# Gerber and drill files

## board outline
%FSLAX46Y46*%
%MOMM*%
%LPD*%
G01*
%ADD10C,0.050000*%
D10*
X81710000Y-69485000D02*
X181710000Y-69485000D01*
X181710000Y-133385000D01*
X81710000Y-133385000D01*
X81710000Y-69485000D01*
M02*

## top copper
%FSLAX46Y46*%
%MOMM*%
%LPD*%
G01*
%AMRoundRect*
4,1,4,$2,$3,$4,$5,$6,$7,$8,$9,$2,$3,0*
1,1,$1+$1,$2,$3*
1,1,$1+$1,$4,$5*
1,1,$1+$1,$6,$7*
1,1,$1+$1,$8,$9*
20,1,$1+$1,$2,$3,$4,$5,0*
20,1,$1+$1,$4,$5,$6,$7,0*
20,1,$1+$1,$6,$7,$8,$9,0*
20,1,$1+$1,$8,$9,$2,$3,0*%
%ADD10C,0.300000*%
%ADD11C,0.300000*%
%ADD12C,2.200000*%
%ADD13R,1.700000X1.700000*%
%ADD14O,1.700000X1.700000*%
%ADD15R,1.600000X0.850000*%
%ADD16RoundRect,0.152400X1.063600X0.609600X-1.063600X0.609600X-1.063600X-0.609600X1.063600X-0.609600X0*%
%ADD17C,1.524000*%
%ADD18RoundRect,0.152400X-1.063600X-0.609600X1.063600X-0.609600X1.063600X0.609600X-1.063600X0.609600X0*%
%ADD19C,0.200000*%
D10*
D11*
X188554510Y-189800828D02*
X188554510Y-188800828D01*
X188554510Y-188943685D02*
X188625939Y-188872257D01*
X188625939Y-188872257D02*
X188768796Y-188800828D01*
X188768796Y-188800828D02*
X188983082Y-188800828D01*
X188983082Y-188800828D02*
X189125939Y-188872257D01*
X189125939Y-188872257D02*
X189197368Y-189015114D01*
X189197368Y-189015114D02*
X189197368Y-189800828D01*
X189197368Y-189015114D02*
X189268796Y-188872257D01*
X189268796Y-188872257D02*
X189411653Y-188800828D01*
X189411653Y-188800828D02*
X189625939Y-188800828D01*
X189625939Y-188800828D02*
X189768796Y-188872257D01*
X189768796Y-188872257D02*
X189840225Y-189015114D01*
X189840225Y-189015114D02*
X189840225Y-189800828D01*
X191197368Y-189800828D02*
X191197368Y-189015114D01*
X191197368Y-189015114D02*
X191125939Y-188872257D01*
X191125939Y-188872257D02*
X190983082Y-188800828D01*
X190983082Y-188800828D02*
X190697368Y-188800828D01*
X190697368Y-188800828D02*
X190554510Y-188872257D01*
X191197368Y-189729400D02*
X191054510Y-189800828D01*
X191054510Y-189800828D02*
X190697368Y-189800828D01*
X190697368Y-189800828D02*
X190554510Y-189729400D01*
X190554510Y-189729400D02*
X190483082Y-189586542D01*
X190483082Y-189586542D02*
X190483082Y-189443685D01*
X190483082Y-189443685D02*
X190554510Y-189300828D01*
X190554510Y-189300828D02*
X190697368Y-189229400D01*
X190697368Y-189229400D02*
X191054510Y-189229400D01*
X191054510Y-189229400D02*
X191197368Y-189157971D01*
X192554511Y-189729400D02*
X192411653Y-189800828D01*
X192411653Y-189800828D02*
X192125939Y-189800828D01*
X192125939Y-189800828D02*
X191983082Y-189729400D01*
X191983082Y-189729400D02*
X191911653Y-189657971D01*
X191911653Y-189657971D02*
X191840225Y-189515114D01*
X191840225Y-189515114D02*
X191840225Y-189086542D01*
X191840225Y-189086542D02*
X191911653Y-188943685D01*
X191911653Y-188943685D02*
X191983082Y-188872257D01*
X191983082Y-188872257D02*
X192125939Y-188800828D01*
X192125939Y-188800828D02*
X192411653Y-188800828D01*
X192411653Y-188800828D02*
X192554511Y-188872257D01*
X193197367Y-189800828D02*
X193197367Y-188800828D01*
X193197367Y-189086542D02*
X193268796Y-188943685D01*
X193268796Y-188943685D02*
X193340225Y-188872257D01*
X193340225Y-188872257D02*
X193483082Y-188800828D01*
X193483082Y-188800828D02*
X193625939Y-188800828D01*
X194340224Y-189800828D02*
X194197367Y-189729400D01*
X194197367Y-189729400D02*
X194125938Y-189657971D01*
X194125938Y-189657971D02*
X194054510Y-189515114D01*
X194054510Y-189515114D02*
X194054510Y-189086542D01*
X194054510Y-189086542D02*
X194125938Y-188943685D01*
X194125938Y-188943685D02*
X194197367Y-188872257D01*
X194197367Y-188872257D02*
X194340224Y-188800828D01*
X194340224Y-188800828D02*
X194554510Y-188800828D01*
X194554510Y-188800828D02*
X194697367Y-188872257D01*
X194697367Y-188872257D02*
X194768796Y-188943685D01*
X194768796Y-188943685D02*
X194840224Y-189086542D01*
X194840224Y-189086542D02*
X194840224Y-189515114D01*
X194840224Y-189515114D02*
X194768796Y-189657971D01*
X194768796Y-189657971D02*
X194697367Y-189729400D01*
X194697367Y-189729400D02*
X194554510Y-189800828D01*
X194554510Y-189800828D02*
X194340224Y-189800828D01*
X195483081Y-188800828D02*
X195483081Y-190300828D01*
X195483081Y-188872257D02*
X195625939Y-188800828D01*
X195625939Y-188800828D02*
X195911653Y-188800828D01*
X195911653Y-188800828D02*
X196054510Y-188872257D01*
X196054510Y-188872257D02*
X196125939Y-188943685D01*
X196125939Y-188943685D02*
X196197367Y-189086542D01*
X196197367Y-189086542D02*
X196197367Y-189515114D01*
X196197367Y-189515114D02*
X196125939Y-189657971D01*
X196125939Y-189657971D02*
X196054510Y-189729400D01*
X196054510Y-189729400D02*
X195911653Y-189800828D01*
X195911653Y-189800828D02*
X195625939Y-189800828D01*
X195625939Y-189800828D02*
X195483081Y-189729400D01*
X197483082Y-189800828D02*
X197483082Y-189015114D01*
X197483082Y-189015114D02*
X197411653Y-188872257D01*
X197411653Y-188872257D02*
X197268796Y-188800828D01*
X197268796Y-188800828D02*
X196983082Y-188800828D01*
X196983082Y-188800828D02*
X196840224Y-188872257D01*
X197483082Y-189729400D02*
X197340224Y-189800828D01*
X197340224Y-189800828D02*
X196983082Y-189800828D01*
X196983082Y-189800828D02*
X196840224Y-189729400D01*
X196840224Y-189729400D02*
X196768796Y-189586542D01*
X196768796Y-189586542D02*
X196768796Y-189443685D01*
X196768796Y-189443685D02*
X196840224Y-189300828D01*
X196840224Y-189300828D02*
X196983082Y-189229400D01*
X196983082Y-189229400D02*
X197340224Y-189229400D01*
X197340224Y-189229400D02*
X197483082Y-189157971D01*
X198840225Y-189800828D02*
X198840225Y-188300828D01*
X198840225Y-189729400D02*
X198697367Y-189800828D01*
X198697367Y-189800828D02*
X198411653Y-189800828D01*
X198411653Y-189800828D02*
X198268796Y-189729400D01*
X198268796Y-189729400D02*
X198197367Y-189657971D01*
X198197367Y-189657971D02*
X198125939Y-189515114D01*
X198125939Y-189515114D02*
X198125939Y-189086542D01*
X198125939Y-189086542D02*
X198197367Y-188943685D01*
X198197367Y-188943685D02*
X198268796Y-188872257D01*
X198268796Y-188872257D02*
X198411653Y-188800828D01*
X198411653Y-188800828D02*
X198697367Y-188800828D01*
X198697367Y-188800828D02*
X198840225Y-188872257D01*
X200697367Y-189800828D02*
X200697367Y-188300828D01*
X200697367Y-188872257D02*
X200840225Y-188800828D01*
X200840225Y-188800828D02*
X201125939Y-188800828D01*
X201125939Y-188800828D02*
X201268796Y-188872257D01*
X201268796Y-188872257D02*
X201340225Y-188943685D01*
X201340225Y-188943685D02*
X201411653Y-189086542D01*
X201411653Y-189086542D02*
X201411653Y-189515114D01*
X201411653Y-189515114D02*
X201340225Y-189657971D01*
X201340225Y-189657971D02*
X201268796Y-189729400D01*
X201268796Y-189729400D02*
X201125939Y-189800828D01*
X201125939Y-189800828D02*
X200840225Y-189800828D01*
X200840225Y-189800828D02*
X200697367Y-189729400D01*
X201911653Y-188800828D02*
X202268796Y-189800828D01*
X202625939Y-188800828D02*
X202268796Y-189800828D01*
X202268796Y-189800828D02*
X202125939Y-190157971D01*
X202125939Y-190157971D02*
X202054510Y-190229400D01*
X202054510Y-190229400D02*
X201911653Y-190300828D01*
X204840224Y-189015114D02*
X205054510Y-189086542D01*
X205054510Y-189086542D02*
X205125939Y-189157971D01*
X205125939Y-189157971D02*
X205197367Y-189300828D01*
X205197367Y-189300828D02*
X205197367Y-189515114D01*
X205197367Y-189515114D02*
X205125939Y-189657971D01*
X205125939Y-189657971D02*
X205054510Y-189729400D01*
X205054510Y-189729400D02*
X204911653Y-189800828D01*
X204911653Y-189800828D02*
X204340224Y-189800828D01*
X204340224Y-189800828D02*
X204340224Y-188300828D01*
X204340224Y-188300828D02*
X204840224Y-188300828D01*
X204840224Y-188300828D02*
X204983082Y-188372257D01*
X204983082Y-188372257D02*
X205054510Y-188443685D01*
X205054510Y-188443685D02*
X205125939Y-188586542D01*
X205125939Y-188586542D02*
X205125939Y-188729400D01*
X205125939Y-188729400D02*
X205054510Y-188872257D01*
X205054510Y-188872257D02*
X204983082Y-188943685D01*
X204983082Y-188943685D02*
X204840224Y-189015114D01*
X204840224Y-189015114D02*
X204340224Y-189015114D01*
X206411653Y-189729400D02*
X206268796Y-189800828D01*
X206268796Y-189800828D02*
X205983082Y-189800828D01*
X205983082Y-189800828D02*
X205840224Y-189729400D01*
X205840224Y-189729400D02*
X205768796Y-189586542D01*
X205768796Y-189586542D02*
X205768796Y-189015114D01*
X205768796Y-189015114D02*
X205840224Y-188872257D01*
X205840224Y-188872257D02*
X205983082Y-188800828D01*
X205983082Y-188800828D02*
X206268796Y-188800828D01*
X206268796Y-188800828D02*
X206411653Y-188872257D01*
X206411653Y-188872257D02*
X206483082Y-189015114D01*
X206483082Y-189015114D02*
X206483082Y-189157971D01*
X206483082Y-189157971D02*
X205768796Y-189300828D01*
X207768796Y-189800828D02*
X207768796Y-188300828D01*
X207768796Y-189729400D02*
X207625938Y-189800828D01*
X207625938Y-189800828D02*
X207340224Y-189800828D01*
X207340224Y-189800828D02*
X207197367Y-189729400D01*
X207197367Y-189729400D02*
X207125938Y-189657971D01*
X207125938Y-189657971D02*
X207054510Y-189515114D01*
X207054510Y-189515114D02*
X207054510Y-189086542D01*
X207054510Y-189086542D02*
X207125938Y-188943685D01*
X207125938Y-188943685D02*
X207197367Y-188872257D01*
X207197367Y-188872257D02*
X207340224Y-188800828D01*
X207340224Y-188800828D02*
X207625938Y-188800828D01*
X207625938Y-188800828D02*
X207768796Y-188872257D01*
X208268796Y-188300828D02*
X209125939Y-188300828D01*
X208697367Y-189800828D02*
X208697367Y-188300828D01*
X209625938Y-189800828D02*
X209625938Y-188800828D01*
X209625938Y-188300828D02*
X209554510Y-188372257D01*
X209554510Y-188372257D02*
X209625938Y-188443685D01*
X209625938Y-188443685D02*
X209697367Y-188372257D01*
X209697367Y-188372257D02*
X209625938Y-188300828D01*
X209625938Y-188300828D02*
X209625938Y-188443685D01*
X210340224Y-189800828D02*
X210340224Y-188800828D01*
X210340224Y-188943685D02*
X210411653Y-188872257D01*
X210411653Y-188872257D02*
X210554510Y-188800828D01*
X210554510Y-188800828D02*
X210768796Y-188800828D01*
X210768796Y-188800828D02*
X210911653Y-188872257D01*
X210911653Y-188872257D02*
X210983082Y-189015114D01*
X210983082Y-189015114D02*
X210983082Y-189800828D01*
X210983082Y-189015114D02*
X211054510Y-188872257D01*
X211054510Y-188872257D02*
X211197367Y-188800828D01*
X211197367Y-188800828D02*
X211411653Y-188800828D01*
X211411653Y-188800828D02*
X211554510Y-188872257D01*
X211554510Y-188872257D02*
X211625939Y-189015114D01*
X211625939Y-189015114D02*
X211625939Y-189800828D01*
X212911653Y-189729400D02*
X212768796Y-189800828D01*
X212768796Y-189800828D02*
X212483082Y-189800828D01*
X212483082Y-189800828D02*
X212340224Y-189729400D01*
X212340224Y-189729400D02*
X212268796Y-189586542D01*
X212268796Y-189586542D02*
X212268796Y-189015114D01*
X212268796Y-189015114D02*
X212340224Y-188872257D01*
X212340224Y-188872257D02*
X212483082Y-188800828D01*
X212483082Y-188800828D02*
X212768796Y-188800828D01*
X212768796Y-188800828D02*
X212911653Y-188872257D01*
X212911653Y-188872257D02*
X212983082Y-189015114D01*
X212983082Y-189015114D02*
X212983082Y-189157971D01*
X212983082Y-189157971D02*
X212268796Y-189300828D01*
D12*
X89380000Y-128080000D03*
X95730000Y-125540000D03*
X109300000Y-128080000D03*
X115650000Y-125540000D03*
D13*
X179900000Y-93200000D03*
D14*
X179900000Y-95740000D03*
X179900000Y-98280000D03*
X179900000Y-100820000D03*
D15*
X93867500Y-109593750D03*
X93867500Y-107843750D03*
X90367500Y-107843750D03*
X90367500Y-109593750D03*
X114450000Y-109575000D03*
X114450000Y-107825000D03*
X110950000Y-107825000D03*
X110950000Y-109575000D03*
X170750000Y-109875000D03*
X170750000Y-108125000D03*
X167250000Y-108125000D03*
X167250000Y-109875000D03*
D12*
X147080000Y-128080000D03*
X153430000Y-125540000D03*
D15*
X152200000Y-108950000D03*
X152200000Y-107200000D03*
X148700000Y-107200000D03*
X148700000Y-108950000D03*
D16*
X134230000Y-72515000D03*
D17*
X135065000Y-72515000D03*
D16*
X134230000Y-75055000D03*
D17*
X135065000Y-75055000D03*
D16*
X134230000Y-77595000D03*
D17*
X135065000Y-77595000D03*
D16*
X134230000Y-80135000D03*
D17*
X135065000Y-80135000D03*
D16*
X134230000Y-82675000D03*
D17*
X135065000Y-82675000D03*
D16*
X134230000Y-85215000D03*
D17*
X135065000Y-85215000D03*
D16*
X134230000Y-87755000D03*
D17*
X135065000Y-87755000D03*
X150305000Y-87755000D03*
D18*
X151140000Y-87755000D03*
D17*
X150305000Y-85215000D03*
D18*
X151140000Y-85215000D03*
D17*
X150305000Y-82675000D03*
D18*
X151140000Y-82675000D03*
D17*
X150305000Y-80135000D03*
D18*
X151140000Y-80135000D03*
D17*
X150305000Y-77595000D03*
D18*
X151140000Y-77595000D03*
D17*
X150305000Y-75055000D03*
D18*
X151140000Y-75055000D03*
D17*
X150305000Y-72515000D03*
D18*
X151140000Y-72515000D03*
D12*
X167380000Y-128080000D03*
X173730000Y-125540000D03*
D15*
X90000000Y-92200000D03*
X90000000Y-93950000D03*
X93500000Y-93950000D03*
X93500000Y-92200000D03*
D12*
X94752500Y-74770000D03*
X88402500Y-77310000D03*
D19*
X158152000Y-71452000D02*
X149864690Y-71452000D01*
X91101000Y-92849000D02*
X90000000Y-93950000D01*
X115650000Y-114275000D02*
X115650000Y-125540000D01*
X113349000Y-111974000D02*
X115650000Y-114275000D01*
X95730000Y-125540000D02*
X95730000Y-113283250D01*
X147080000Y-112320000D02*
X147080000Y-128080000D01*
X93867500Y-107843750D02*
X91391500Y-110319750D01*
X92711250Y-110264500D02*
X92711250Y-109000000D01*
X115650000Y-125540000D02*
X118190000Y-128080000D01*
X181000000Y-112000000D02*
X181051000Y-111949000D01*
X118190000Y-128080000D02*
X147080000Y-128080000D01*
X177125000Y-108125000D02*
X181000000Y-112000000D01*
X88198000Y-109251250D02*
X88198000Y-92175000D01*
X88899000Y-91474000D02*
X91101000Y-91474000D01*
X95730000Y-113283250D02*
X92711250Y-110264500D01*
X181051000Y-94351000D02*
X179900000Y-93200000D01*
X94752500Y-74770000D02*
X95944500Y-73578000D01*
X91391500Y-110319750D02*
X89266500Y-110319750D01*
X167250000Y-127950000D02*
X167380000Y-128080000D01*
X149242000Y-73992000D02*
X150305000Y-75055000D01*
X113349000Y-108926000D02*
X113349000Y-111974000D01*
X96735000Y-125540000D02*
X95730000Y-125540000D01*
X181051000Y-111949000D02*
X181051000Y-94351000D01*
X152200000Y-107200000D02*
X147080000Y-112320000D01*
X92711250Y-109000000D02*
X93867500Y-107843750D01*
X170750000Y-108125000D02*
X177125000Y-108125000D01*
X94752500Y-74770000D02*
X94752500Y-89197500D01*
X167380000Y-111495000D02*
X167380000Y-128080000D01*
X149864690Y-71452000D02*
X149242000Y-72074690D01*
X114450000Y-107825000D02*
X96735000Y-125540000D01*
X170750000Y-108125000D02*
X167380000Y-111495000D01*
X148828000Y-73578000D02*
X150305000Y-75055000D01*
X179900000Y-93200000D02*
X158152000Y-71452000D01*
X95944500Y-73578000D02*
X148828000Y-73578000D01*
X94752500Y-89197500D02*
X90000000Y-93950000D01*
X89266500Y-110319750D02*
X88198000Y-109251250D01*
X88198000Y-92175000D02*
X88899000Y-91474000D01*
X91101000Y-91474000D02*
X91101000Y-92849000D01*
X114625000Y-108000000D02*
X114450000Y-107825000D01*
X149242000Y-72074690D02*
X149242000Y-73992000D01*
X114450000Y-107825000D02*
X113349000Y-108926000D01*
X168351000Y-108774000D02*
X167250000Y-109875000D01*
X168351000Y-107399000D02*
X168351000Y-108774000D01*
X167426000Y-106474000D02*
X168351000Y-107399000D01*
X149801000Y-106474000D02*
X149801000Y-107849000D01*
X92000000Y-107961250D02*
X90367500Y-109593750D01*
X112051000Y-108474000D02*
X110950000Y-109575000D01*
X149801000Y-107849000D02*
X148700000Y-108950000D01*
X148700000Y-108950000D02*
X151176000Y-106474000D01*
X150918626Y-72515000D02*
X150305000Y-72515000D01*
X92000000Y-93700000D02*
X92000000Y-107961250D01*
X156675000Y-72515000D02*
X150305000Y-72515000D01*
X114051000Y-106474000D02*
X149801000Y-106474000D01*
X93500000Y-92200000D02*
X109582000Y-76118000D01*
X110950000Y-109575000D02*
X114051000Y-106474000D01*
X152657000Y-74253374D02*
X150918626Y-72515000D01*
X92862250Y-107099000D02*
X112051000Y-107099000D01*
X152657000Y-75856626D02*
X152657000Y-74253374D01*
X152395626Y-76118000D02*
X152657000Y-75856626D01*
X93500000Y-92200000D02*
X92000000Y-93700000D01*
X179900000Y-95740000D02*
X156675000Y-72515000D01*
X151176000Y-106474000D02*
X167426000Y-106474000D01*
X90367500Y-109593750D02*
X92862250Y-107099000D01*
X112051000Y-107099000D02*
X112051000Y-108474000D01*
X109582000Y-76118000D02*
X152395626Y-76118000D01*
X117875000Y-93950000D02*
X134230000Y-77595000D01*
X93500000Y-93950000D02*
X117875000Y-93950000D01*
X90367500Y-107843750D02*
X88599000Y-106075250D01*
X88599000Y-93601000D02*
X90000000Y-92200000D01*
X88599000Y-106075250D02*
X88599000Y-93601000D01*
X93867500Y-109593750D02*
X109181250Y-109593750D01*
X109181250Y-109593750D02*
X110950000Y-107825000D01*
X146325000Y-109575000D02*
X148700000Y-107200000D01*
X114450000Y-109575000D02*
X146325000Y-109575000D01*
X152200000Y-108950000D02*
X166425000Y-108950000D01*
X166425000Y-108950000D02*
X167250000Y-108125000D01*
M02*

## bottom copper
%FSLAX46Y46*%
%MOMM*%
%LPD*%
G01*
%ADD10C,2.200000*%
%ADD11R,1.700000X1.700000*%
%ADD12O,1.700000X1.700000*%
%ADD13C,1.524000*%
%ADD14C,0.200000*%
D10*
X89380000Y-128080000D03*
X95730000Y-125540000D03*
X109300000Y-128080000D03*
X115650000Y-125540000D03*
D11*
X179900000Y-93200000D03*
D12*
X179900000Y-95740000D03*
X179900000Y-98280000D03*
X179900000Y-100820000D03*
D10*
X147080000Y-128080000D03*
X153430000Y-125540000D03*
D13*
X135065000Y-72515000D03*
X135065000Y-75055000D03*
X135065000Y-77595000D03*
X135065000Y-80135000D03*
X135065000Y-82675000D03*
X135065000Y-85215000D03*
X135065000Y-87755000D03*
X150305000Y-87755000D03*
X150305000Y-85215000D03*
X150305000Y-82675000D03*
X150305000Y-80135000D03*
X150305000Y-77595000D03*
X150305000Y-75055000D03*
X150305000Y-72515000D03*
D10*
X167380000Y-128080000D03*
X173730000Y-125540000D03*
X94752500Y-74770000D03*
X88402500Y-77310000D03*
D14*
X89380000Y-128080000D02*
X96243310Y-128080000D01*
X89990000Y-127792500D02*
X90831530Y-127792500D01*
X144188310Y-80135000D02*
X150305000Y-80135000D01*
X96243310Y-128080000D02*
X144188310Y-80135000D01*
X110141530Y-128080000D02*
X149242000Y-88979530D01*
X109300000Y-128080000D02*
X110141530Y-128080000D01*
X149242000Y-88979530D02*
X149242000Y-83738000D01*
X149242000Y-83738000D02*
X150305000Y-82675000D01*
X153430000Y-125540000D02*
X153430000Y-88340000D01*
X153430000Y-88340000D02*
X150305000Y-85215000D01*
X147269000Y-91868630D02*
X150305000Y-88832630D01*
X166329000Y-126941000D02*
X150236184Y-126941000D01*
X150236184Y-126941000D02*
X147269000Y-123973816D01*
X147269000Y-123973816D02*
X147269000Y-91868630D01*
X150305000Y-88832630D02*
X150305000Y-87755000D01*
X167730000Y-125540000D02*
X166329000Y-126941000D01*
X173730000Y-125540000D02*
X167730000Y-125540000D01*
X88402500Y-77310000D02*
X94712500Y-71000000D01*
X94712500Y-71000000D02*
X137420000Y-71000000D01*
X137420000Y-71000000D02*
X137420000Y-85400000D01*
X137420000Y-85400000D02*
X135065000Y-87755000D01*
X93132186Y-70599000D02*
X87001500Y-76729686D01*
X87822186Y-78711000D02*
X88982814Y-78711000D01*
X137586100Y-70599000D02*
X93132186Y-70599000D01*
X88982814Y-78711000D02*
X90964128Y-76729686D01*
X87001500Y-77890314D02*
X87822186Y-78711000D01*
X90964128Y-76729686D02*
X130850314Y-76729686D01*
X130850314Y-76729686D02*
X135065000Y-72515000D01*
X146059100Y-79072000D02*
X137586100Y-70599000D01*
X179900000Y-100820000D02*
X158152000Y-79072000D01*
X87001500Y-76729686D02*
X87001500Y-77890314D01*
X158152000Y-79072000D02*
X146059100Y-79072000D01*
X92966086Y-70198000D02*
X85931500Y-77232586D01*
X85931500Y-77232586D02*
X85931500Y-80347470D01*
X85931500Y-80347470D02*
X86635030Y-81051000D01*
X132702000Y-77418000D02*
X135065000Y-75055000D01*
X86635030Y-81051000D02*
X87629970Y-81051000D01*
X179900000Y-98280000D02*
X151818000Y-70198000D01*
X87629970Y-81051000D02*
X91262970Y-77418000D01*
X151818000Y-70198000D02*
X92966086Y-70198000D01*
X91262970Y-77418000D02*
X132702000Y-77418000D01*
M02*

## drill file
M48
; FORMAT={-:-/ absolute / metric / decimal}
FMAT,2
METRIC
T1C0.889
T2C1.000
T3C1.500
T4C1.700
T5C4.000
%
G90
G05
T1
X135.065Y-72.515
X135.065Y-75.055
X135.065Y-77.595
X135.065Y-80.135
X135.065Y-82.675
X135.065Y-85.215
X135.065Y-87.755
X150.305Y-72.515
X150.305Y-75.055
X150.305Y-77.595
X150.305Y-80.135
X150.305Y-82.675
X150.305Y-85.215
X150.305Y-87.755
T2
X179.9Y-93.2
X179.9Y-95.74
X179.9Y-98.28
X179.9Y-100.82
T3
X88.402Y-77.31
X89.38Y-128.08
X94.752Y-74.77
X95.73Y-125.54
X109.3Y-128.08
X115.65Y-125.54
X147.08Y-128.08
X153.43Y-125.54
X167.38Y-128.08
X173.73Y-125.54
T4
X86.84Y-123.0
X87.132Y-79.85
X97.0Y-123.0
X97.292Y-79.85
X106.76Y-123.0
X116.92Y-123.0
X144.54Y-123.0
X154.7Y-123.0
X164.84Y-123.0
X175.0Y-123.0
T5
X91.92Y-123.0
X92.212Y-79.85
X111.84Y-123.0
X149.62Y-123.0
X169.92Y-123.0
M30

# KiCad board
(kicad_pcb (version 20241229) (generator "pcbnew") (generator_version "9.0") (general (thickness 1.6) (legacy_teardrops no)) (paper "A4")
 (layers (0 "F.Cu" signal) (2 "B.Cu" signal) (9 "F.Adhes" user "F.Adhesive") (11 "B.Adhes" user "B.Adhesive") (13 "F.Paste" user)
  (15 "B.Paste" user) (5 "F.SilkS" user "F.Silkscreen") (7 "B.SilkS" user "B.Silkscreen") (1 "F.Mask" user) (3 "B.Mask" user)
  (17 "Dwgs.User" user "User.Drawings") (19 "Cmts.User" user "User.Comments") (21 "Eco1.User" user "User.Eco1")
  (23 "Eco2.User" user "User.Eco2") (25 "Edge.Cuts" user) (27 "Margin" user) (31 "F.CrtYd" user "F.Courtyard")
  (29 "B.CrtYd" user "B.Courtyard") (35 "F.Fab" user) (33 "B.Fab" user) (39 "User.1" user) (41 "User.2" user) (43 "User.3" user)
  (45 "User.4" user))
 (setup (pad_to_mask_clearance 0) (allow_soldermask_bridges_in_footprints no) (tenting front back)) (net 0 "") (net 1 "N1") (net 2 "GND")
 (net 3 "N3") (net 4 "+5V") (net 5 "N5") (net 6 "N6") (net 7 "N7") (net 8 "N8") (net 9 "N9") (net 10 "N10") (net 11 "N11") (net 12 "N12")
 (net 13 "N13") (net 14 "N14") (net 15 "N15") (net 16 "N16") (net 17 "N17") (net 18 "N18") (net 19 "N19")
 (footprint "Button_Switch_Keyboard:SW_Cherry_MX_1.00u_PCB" (layer "F.Cu") (at 89.38 128.08 180)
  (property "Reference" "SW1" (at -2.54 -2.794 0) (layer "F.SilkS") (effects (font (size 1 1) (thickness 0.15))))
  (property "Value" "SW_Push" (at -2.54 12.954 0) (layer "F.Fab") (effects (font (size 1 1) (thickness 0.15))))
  (pad "" np_thru_hole circle (at -7.62 5.08 180) (size 1.7 1.7) (drill 1.7) (layers "*.Cu" "*.Mask"))
  (pad "" np_thru_hole circle (at -2.54 5.08 180) (size 4 4) (drill 4) (layers "*.Cu" "*.Mask"))
  (pad "" np_thru_hole circle (at 2.54 5.08 180) (size 1.7 1.7) (drill 1.7) (layers "*.Cu" "*.Mask"))
  (pad "1" thru_hole circle (at 0 0 180) (size 2.2 2.2) (drill 1.5) (layers "*.Cu" "*.Mask") (remove_unused_layers no) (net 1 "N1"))
  (pad "2" thru_hole circle (at -6.35 2.54 180) (size 2.2 2.2) (drill 1.5) (layers "*.Cu" "*.Mask") (remove_unused_layers no) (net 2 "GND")))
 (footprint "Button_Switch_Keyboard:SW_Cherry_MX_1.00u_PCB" (layer "F.Cu") (at 109.3 128.08 180)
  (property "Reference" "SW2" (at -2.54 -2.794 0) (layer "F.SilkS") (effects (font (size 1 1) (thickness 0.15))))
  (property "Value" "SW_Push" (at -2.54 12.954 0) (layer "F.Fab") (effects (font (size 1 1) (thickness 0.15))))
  (pad "" np_thru_hole circle (at -7.62 5.08 180) (size 1.7 1.7) (drill 1.7) (layers "*.Cu" "*.Mask"))
  (pad "" np_thru_hole circle (at -2.54 5.08 180) (size 4 4) (drill 4) (layers "*.Cu" "*.Mask"))
  (pad "" np_thru_hole circle (at 2.54 5.08 180) (size 1.7 1.7) (drill 1.7) (layers "*.Cu" "*.Mask"))
  (pad "1" thru_hole circle (at 0 0 180) (size 2.2 2.2) (drill 1.5) (layers "*.Cu" "*.Mask") (remove_unused_layers no) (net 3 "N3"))
  (pad "2" thru_hole circle (at -6.35 2.54 180) (size 2.2 2.2) (drill 1.5) (layers "*.Cu" "*.Mask") (remove_unused_layers no) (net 2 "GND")))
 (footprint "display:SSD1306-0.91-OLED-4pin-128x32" (layer "F.Cu") (at 143.4 91.01)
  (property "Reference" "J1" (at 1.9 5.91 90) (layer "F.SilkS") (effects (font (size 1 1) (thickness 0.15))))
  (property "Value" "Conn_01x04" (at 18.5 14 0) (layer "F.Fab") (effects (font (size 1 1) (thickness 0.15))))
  (pad "1" thru_hole rect (at 36.5 2.19) (size 1.7 1.7) (drill 1) (layers "*.Cu" "*.Mask") (remove_unused_layers no) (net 2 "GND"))
  (pad "2" thru_hole oval (at 36.5 4.73) (size 1.7 1.7) (drill 1) (layers "*.Cu" "*.Mask") (remove_unused_layers no) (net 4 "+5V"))
  (pad "3" thru_hole oval (at 36.5 7.27) (size 1.7 1.7) (drill 1) (layers "*.Cu" "*.Mask") (remove_unused_layers no) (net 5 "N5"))
  (pad "4" thru_hole oval (at 36.5 9.81) (size 1.7 1.7) (drill 1) (layers "*.Cu" "*.Mask") (remove_unused_layers no) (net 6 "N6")))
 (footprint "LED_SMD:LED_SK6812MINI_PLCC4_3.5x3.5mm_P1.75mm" (layer "F.Cu") (at 92.1175 108.71875 180)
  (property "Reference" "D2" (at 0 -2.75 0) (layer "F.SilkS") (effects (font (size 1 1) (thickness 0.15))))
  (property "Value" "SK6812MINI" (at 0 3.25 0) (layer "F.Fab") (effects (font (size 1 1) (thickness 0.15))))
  (pad "1" smd rect (at -1.75 -0.875 180) (size 1.6 0.85) (layers "F.Cu" "F.Mask" "F.Paste") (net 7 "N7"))
  (pad "2" smd rect (at -1.75 0.875 180) (size 1.6 0.85) (layers "F.Cu" "F.Mask" "F.Paste") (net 2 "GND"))
  (pad "3" smd rect (at 1.75 0.875 180) (size 1.6 0.85) (layers "F.Cu" "F.Mask" "F.Paste") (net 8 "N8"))
  (pad "4" smd rect (at 1.75 -0.875 180) (size 1.6 0.85) (layers "F.Cu" "F.Mask" "F.Paste") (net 4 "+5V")))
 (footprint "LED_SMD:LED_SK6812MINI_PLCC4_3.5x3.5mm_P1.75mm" (layer "F.Cu") (at 112.7 108.7 180)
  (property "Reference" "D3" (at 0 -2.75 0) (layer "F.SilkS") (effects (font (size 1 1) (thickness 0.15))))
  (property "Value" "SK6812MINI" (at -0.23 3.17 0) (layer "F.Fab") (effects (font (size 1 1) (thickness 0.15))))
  (pad "1" smd rect (at -1.75 -0.875 180) (size 1.6 0.85) (layers "F.Cu" "F.Mask" "F.Paste") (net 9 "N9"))
  (pad "2" smd rect (at -1.75 0.875 180) (size 1.6 0.85) (layers "F.Cu" "F.Mask" "F.Paste") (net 2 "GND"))
  (pad "3" smd rect (at 1.75 0.875 180) (size 1.6 0.85) (layers "F.Cu" "F.Mask" "F.Paste") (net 7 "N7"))
  (pad "4" smd rect (at 1.75 -0.875 180) (size 1.6 0.85) (layers "F.Cu" "F.Mask" "F.Paste") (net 4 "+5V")))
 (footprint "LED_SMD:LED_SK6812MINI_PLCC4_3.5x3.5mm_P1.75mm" (layer "F.Cu") (at 169 109 180)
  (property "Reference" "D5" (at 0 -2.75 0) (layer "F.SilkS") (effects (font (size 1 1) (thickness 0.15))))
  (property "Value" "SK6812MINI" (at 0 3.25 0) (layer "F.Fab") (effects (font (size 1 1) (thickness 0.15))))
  (pad "1" smd rect (at -1.75 -0.875 180) (size 1.6 0.85) (layers "F.Cu" "F.Mask" "F.Paste") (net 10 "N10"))
  (pad "2" smd rect (at -1.75 0.875 180) (size 1.6 0.85) (layers "F.Cu" "F.Mask" "F.Paste") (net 2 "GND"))
  (pad "3" smd rect (at 1.75 0.875 180) (size 1.6 0.85) (layers "F.Cu" "F.Mask" "F.Paste") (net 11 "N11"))
  (pad "4" smd rect (at 1.75 -0.875 180) (size 1.6 0.85) (layers "F.Cu" "F.Mask" "F.Paste") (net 4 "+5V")))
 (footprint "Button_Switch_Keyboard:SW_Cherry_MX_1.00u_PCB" (layer "F.Cu") (at 147.08 128.08 180)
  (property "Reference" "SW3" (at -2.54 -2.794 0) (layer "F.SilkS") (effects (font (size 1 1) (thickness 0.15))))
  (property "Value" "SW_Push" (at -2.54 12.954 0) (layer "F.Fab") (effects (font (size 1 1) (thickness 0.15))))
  (pad "" np_thru_hole circle (at -7.62 5.08 180) (size 1.7 1.7) (drill 1.7) (layers "*.Cu" "*.Mask"))
  (pad "" np_thru_hole circle (at -2.54 5.08 180) (size 4 4) (drill 4) (layers "*.Cu" "*.Mask"))
  (pad "" np_thru_hole circle (at 2.54 5.08 180) (size 1.7 1.7) (drill 1.7) (layers "*.Cu" "*.Mask"))
  (pad "1" thru_hole circle (at 0 0 180) (size 2.2 2.2) (drill 1.5) (layers "*.Cu" "*.Mask") (remove_unused_layers no) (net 2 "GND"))
  (pad "2" thru_hole circle (at -6.35 2.54 180) (size 2.2 2.2) (drill 1.5) (layers "*.Cu" "*.Mask") (remove_unused_layers no) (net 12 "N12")))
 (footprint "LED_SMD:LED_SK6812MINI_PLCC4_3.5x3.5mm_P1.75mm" (layer "F.Cu") (at 150.45 108.075 180)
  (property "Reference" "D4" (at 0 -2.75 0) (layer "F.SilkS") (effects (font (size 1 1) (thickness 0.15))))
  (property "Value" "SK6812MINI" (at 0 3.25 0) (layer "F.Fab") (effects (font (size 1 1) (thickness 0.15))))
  (pad "1" smd rect (at -1.75 -0.875 180) (size 1.6 0.85) (layers "F.Cu" "F.Mask" "F.Paste") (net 11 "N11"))
  (pad "2" smd rect (at -1.75 0.875 180) (size 1.6 0.85) (layers "F.Cu" "F.Mask" "F.Paste") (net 2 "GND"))
  (pad "3" smd rect (at 1.75 0.875 180) (size 1.6 0.85) (layers "F.Cu" "F.Mask" "F.Paste") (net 9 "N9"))
  (pad "4" smd rect (at 1.75 -0.875 180) (size 1.6 0.85) (layers "F.Cu" "F.Mask" "F.Paste") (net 4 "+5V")))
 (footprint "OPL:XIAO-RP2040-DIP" (layer "F.Cu") (at 142.685 80.135)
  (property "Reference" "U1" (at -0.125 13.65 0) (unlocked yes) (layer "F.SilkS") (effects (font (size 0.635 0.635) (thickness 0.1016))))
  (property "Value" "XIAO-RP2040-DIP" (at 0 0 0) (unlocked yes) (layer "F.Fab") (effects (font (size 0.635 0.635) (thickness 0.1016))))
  (pad "1" smd roundrect (at -8.455 -7.62 180) (size 2.432 1.524) (layers "F.Cu" "F.Mask") (roundrect_rratio 0.1) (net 6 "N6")
   (thermal_bridge_angle 45))
  (pad "1" thru_hole circle (at -7.62 -7.62 180) (size 1.524 1.524) (drill 0.889) (layers "*.Cu" "*.Mask") (remove_unused_layers no)
   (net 6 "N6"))
  (pad "2" smd roundrect (at -8.455 -5.08 180) (size 2.432 1.524) (layers "F.Cu" "F.Mask") (roundrect_rratio 0.1) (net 5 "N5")
   (thermal_bridge_angle 45))
  (pad "2" thru_hole circle (at -7.62 -5.08 180) (size 1.524 1.524) (drill 0.889) (layers "*.Cu" "*.Mask") (remove_unused_layers no)
   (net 5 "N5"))
  (pad "3" smd roundrect (at -8.455 -2.54 180) (size 2.432 1.524) (layers "F.Cu" "F.Mask") (roundrect_rratio 0.1) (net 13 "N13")
   (thermal_bridge_angle 45))
  (pad "3" thru_hole circle (at -7.62 -2.54 180) (size 1.524 1.524) (drill 0.889) (layers "*.Cu" "*.Mask") (remove_unused_layers no)
   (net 13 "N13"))
  (pad "4" smd roundrect (at -8.455 0 180) (size 2.432 1.524) (layers "F.Cu" "F.Mask") (roundrect_rratio 0.1) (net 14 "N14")
   (thermal_bridge_angle 45))
  (pad "4" thru_hole circle (at -7.62 0 180) (size 1.524 1.524) (drill 0.889) (layers "*.Cu" "*.Mask") (remove_unused_layers no)
   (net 14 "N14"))
  (pad "5" smd roundrect (at -8.455 2.54 180) (size 2.432 1.524) (layers "F.Cu" "F.Mask") (roundrect_rratio 0.1) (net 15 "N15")
   (thermal_bridge_angle 45))
  (pad "5" thru_hole circle (at -7.62 2.54 180) (size 1.524 1.524) (drill 0.889) (layers "*.Cu" "*.Mask") (remove_unused_layers no)
   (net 15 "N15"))
  (pad "6" smd roundrect (at -8.455 5.08 180) (size 2.432 1.524) (layers "F.Cu" "F.Mask") (roundrect_rratio 0.1) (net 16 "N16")
   (thermal_bridge_angle 45))
  (pad "6" thru_hole circle (at -7.62 5.08 180) (size 1.524 1.524) (drill 0.889) (layers "*.Cu" "*.Mask") (remove_unused_layers no)
   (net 16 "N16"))
  (pad "7" smd roundrect (at -8.455 7.62 180) (size 2.432 1.524) (layers "F.Cu" "F.Mask") (roundrect_rratio 0.1) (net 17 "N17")
   (thermal_bridge_angle 45))
  (pad "7" thru_hole circle (at -7.62 7.62 180) (size 1.524 1.524) (drill 0.889) (layers "*.Cu" "*.Mask") (remove_unused_layers no)
   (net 17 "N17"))
  (pad "8" thru_hole circle (at 7.62 7.62) (size 1.524 1.524) (drill 0.889) (layers "*.Cu" "*.Mask") (remove_unused_layers no)
   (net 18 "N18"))
  (pad "8" smd roundrect (at 8.455 7.62) (size 2.432 1.524) (layers "F.Cu" "F.Mask") (roundrect_rratio 0.1) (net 18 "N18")
   (thermal_bridge_angle 45))
  (pad "9" thru_hole circle (at 7.62 5.08) (size 1.524 1.524) (drill 0.889) (layers "*.Cu" "*.Mask") (remove_unused_layers no)
   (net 12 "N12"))
  (pad "9" smd roundrect (at 8.455 5.08) (size 2.432 1.524) (layers "F.Cu" "F.Mask") (roundrect_rratio 0.1) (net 12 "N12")
   (thermal_bridge_angle 45))
  (pad "10" thru_hole circle (at 7.62 2.54) (size 1.524 1.524) (drill 0.889) (layers "*.Cu" "*.Mask") (remove_unused_layers no) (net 3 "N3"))
  (pad "10" smd roundrect (at 8.455 2.54) (size 2.432 1.524) (layers "F.Cu" "F.Mask") (roundrect_rratio 0.1) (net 3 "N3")
   (thermal_bridge_angle 45))
  (pad "11" thru_hole circle (at 7.62 0) (size 1.524 1.524) (drill 0.889) (layers "*.Cu" "*.Mask") (remove_unused_layers no) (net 1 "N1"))
  (pad "11" smd roundrect (at 8.455 0) (size 2.432 1.524) (layers "F.Cu" "F.Mask") (roundrect_rratio 0.1) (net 1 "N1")
   (thermal_bridge_angle 45))
  (pad "12" thru_hole circle (at 7.62 -2.54) (size 1.524 1.524) (drill 0.889) (layers "*.Cu" "*.Mask") (remove_unused_layers no)
   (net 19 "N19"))
  (pad "12" smd roundrect (at 8.455 -2.54) (size 2.432 1.524) (layers "F.Cu" "F.Mask") (roundrect_rratio 0.1) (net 19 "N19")
   (thermal_bridge_angle 45))
  (pad "13" thru_hole circle (at 7.62 -5.08) (size 1.524 1.524) (drill 0.889) (layers "*.Cu" "*.Mask") (remove_unused_layers no)
   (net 2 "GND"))
  (pad "13" smd roundrect (at 8.455 -5.08) (size 2.432 1.524) (layers "F.Cu" "F.Mask") (roundrect_rratio 0.1) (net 2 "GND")
   (thermal_bridge_angle 45))
  (pad "14" thru_hole circle (at 7.62 -7.62) (size 1.524 1.524) (drill 0.889) (layers "*.Cu" "*.Mask") (remove_unused_layers no)
   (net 4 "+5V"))
  (pad "14" smd roundrect (at 8.455 -7.62) (size 2.432 1.524) (layers "F.Cu" "F.Mask") (roundrect_rratio 0.1) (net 4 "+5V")
   (thermal_bridge_angle 45)))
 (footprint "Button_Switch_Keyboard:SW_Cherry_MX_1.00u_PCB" (layer "F.Cu") (at 167.38 128.08 180)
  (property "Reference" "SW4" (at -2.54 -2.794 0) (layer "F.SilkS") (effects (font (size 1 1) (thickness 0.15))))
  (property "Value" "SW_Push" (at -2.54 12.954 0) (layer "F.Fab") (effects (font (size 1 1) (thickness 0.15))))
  (pad "" np_thru_hole circle (at -7.62 5.08 180) (size 1.7 1.7) (drill 1.7) (layers "*.Cu" "*.Mask"))
  (pad "" np_thru_hole circle (at -2.54 5.08 180) (size 4 4) (drill 4) (layers "*.Cu" "*.Mask"))
  (pad "" np_thru_hole circle (at 2.54 5.08 180) (size 1.7 1.7) (drill 1.7) (layers "*.Cu" "*.Mask"))
  (pad "1" thru_hole circle (at 0 0 180) (size 2.2 2.2) (drill 1.5) (layers "*.Cu" "*.Mask") (remove_unused_layers no) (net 2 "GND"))
  (pad "2" thru_hole circle (at -6.35 2.54 180) (size 2.2 2.2) (drill 1.5) (layers "*.Cu" "*.Mask") (remove_unused_layers no) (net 18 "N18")))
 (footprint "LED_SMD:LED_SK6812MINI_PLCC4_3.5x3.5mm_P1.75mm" (layer "F.Cu") (at 91.75 93.075)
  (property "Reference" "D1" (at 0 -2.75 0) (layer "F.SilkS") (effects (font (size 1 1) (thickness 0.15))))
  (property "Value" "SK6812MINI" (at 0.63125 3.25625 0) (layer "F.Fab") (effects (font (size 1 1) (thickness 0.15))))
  (pad "1" smd rect (at -1.75 -0.875) (size 1.6 0.85) (layers "F.Cu" "F.Mask" "F.Paste") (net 8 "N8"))
  (pad "2" smd rect (at -1.75 0.875) (size 1.6 0.85) (layers "F.Cu" "F.Mask" "F.Paste") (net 2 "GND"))
  (pad "3" smd rect (at 1.75 0.875) (size 1.6 0.85) (layers "F.Cu" "F.Mask" "F.Paste") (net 13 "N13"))
  (pad "4" smd rect (at 1.75 -0.875) (size 1.6 0.85) (layers "F.Cu" "F.Mask" "F.Paste") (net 4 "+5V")))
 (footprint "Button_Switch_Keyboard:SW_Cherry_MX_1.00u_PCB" (layer "F.Cu") (at 94.7525 74.77)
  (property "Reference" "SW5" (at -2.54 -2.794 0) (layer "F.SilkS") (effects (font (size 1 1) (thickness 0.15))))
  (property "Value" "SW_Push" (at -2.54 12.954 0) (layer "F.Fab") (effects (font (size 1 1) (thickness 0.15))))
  (pad "" np_thru_hole circle (at -7.62 5.08) (size 1.7 1.7) (drill 1.7) (layers "*.Cu" "*.Mask"))
  (pad "" np_thru_hole circle (at -2.54 5.08) (size 4 4) (drill 4) (layers "*.Cu" "*.Mask"))
  (pad "" np_thru_hole circle (at 2.54 5.08) (size 1.7 1.7) (drill 1.7) (layers "*.Cu" "*.Mask"))
  (pad "1" thru_hole circle (at 0 0) (size 2.2 2.2) (drill 1.5) (layers "*.Cu" "*.Mask") (remove_unused_layers no) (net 2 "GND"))
  (pad "2" thru_hole circle (at -6.35 2.54) (size 2.2 2.2) (drill 1.5) (layers "*.Cu" "*.Mask") (remove_unused_layers no) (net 17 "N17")))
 (gr_rect (start 81.71 69.485) (end 181.71 133.385) (stroke (width 0.05) (type solid)) (fill no) (layer "Edge.Cuts"))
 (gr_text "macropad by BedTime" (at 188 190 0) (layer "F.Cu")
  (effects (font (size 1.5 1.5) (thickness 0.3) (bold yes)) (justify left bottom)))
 (segment (start 158.152 71.452) (end 149.86469 71.452) (width 0.2) (layer "F.Cu") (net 2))
 (segment (start 91.101 92.849) (end 90 93.95) (width 0.2) (layer "F.Cu") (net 2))
 (segment (start 115.65 114.275) (end 115.65 125.54) (width 0.2) (layer "F.Cu") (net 2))
 (segment (start 113.349 111.974) (end 115.65 114.275) (width 0.2) (layer "F.Cu") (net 2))
 (segment (start 95.73 125.54) (end 95.73 113.28325) (width 0.2) (layer "F.Cu") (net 2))
 (segment (start 147.08 112.32) (end 147.08 128.08) (width 0.2) (layer "F.Cu") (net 2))
 (segment (start 93.8675 107.84375) (end 91.3915 110.31975) (width 0.2) (layer "F.Cu") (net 2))
 (segment (start 92.71125 110.2645) (end 92.71125 109) (width 0.2) (layer "F.Cu") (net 2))
 (segment (start 115.65 125.54) (end 118.19 128.08) (width 0.2) (layer "F.Cu") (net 2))
 (segment (start 181 112) (end 181.051 111.949) (width 0.2) (layer "F.Cu") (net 2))
 (segment (start 118.19 128.08) (end 147.08 128.08) (width 0.2) (layer "F.Cu") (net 2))
 (segment (start 177.125 108.125) (end 181 112) (width 0.2) (layer "F.Cu") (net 2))
 (segment (start 88.198 109.25125) (end 88.198 92.175) (width 0.2) (layer "F.Cu") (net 2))
 (segment (start 88.899 91.474) (end 91.101 91.474) (width 0.2) (layer "F.Cu") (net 2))
 (segment (start 95.73 113.28325) (end 92.71125 110.2645) (width 0.2) (layer "F.Cu") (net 2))
 (segment (start 181.051 94.351) (end 179.9 93.2) (width 0.2) (layer "F.Cu") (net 2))
 (segment (start 94.7525 74.77) (end 95.9445 73.578) (width 0.2) (layer "F.Cu") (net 2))
 (segment (start 91.3915 110.31975) (end 89.2665 110.31975) (width 0.2) (layer "F.Cu") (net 2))
 (segment (start 167.25 127.95) (end 167.38 128.08) (width 0.2) (layer "F.Cu") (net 2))
 (segment (start 149.242 73.992) (end 150.305 75.055) (width 0.2) (layer "F.Cu") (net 2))
 (segment (start 113.349 108.926) (end 113.349 111.974) (width 0.2) (layer "F.Cu") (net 2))
 (segment (start 96.735 125.54) (end 95.73 125.54) (width 0.2) (layer "F.Cu") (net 2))
 (segment (start 181.051 111.949) (end 181.051 94.351) (width 0.2) (layer "F.Cu") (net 2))
 (segment (start 152.2 107.2) (end 147.08 112.32) (width 0.2) (layer "F.Cu") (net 2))
 (segment (start 92.71125 109) (end 93.8675 107.84375) (width 0.2) (layer "F.Cu") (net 2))
 (segment (start 170.75 108.125) (end 177.125 108.125) (width 0.2) (layer "F.Cu") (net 2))
 (segment (start 94.7525 74.77) (end 94.7525 89.1975) (width 0.2) (layer "F.Cu") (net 2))
 (segment (start 167.38 111.495) (end 167.38 128.08) (width 0.2) (layer "F.Cu") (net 2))
 (segment (start 149.86469 71.452) (end 149.242 72.07469) (width 0.2) (layer "F.Cu") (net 2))
 (segment (start 114.45 107.825) (end 96.735 125.54) (width 0.2) (layer "F.Cu") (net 2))
 (segment (start 170.75 108.125) (end 167.38 111.495) (width 0.2) (layer "F.Cu") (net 2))
 (segment (start 148.828 73.578) (end 150.305 75.055) (width 0.2) (layer "F.Cu") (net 2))
 (segment (start 179.9 93.2) (end 158.152 71.452) (width 0.2) (layer "F.Cu") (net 2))
 (segment (start 95.9445 73.578) (end 148.828 73.578) (width 0.2) (layer "F.Cu") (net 2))
 (segment (start 94.7525 89.1975) (end 90 93.95) (width 0.2) (layer "F.Cu") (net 2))
 (segment (start 89.2665 110.31975) (end 88.198 109.25125) (width 0.2) (layer "F.Cu") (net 2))
 (segment (start 88.198 92.175) (end 88.899 91.474) (width 0.2) (layer "F.Cu") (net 2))
 (segment (start 91.101 91.474) (end 91.101 92.849) (width 0.2) (layer "F.Cu") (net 2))
 (segment (start 114.625 108) (end 114.45 107.825) (width 0.2) (layer "F.Cu") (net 2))
 (segment (start 149.242 72.07469) (end 149.242 73.992) (width 0.2) (layer "F.Cu") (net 2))
 (segment (start 114.45 107.825) (end 113.349 108.926) (width 0.2) (layer "F.Cu") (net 2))
 (segment (start 168.351 108.774) (end 167.25 109.875) (width 0.2) (layer "F.Cu") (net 4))
 (segment (start 168.351 107.399) (end 168.351 108.774) (width 0.2) (layer "F.Cu") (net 4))
 (segment (start 167.426 106.474) (end 168.351 107.399) (width 0.2) (layer "F.Cu") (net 4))
 (segment (start 149.801 106.474) (end 149.801 107.849) (width 0.2) (layer "F.Cu") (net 4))
 (segment (start 92 107.96125) (end 90.3675 109.59375) (width 0.2) (layer "F.Cu") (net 4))
 (segment (start 112.051 108.474) (end 110.95 109.575) (width 0.2) (layer "F.Cu") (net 4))
 (segment (start 149.801 107.849) (end 148.7 108.95) (width 0.2) (layer "F.Cu") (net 4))
 (segment (start 148.7 108.95) (end 151.176 106.474) (width 0.2) (layer "F.Cu") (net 4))
 (segment (start 150.918626 72.515) (end 150.305 72.515) (width 0.2) (layer "F.Cu") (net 4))
 (segment (start 92 93.7) (end 92 107.96125) (width 0.2) (layer "F.Cu") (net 4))
 (segment (start 156.675 72.515) (end 150.305 72.515) (width 0.2) (layer "F.Cu") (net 4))
 (segment (start 114.051 106.474) (end 149.801 106.474) (width 0.2) (layer "F.Cu") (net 4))
 (segment (start 93.5 92.2) (end 109.582 76.118) (width 0.2) (layer "F.Cu") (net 4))
 (segment (start 110.95 109.575) (end 114.051 106.474) (width 0.2) (layer "F.Cu") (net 4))
 (segment (start 152.657 74.253374) (end 150.918626 72.515) (width 0.2) (layer "F.Cu") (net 4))
 (segment (start 92.86225 107.099) (end 112.051 107.099) (width 0.2) (layer "F.Cu") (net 4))
 (segment (start 152.657 75.856626) (end 152.657 74.253374) (width 0.2) (layer "F.Cu") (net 4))
 (segment (start 152.395626 76.118) (end 152.657 75.856626) (width 0.2) (layer "F.Cu") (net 4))
 (segment (start 93.5 92.2) (end 92 93.7) (width 0.2) (layer "F.Cu") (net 4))
 (segment (start 179.9 95.74) (end 156.675 72.515) (width 0.2) (layer "F.Cu") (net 4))
 (segment (start 151.176 106.474) (end 167.426 106.474) (width 0.2) (layer "F.Cu") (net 4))
 (segment (start 90.3675 109.59375) (end 92.86225 107.099) (width 0.2) (layer "F.Cu") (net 4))
 (segment (start 112.051 107.099) (end 112.051 108.474) (width 0.2) (layer "F.Cu") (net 4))
 (segment (start 109.582 76.118) (end 152.395626 76.118) (width 0.2) (layer "F.Cu") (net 4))
 (segment (start 117.875 93.95) (end 134.23 77.595) (width 0.2) (layer "F.Cu") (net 13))
 (segment (start 93.5 93.95) (end 117.875 93.95) (width 0.2) (layer "F.Cu") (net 13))
 (segment (start 90.3675 107.84375) (end 88.599 106.07525) (width 0.2) (layer "F.Cu") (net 8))
 (segment (start 88.599 93.601) (end 90 92.2) (width 0.2) (layer "F.Cu") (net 8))
 (segment (start 88.599 106.07525) (end 88.599 93.601) (width 0.2) (layer "F.Cu") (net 8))
 (segment (start 93.8675 109.59375) (end 109.18125 109.59375) (width 0.2) (layer "F.Cu") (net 7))
 (segment (start 109.18125 109.59375) (end 110.95 107.825) (width 0.2) (layer "F.Cu") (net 7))
 (segment (start 89.38 128.08) (end 96.24331 128.08) (width 0.2) (layer "B.Cu") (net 1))
 (segment (start 89.99 127.7925) (end 90.83153 127.7925) (width 0.2) (layer "B.Cu") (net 1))
 (segment (start 144.18831 80.135) (end 150.305 80.135) (width 0.2) (layer "B.Cu") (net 1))
 (segment (start 96.24331 128.08) (end 144.18831 80.135) (width 0.2) (layer "B.Cu") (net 1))
 (segment (start 110.14153 128.08) (end 149.242 88.97953) (width 0.2) (layer "B.Cu") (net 3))
 (segment (start 109.3 128.08) (end 110.14153 128.08) (width 0.2) (layer "B.Cu") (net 3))
 (segment (start 149.242 88.97953) (end 149.242 83.738) (width 0.2) (layer "B.Cu") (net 3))
 (segment (start 149.242 83.738) (end 150.305 82.675) (width 0.2) (layer "B.Cu") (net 3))
 (segment (start 153.43 125.54) (end 153.43 88.34) (width 0.2) (layer "B.Cu") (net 12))
 (segment (start 153.43 88.34) (end 150.305 85.215) (width 0.2) (layer "B.Cu") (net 12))
 (segment (start 147.269 91.86863) (end 150.305 88.83263) (width 0.2) (layer "B.Cu") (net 18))
 (segment (start 166.329 126.941) (end 150.236184 126.941) (width 0.2) (layer "B.Cu") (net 18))
 (segment (start 150.236184 126.941) (end 147.269 123.973816) (width 0.2) (layer "B.Cu") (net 18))
 (segment (start 147.269 123.973816) (end 147.269 91.86863) (width 0.2) (layer "B.Cu") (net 18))
 (segment (start 150.305 88.83263) (end 150.305 87.755) (width 0.2) (layer "B.Cu") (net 18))
 (segment (start 167.73 125.54) (end 166.329 126.941) (width 0.2) (layer "B.Cu") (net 18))
 (segment (start 173.73 125.54) (end 167.73 125.54) (width 0.2) (layer "B.Cu") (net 18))
 (segment (start 88.4025 77.31) (end 94.7125 71) (width 0.2) (layer "B.Cu") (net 17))
 (segment (start 94.7125 71) (end 137.42 71) (width 0.2) (layer "B.Cu") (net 17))
 (segment (start 137.42 71) (end 137.42 85.4) (width 0.2) (layer "B.Cu") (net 17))
 (segment (start 137.42 85.4) (end 135.065 87.755) (width 0.2) (layer "B.Cu") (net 17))
 (segment (start 146.325 109.575) (end 148.7 107.2) (width 0.2) (layer "F.Cu") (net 9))
 (segment (start 114.45 109.575) (end 146.325 109.575) (width 0.2) (layer "F.Cu") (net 9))
 (segment (start 152.2 108.95) (end 166.425 108.95) (width 0.2) (layer "F.Cu") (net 11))
 (segment (start 166.425 108.95) (end 167.25 108.125) (width 0.2) (layer "F.Cu") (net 11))
 (segment (start 93.132186 70.599) (end 87.0015 76.729686) (width 0.2) (layer "B.Cu") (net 6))
 (segment (start 87.822186 78.711) (end 88.982814 78.711) (width 0.2) (layer "B.Cu") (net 6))
 (segment (start 137.5861 70.599) (end 93.132186 70.599) (width 0.2) (layer "B.Cu") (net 6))
 (segment (start 88.982814 78.711) (end 90.964128 76.729686) (width 0.2) (layer "B.Cu") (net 6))
 (segment (start 87.0015 77.890314) (end 87.822186 78.711) (width 0.2) (layer "B.Cu") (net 6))
 (segment (start 90.964128 76.729686) (end 130.850314 76.729686) (width 0.2) (layer "B.Cu") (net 6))
 (segment (start 130.850314 76.729686) (end 135.065 72.515) (width 0.2) (layer "B.Cu") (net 6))
 (segment (start 146.0591 79.072) (end 137.5861 70.599) (width 0.2) (layer "B.Cu") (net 6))
 (segment (start 179.9 100.82) (end 158.152 79.072) (width 0.2) (layer "B.Cu") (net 6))
 (segment (start 87.0015 76.729686) (end 87.0015 77.890314) (width 0.2) (layer "B.Cu") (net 6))
 (segment (start 158.152 79.072) (end 146.0591 79.072) (width 0.2) (layer "B.Cu") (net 6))
 (segment (start 92.966086 70.198) (end 85.9315 77.232586) (width 0.2) (layer "B.Cu") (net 5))
 (segment (start 85.9315 77.232586) (end 85.9315 80.34747) (width 0.2) (layer "B.Cu") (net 5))
 (segment (start 85.9315 80.34747) (end 86.63503 81.051) (width 0.2) (layer "B.Cu") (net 5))
 (segment (start 132.702 77.418) (end 135.065 75.055) (width 0.2) (layer "B.Cu") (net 5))
 (segment (start 86.63503 81.051) (end 87.62997 81.051) (width 0.2) (layer "B.Cu") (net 5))
 (segment (start 179.9 98.28) (end 151.818 70.198) (width 0.2) (layer "B.Cu") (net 5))
 (segment (start 87.62997 81.051) (end 91.26297 77.418) (width 0.2) (layer "B.Cu") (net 5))
 (segment (start 151.818 70.198) (end 92.966086 70.198) (width 0.2) (layer "B.Cu") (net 5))
 (segment (start 91.26297 77.418) (end 132.702 77.418) (width 0.2) (layer "B.Cu") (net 5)))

